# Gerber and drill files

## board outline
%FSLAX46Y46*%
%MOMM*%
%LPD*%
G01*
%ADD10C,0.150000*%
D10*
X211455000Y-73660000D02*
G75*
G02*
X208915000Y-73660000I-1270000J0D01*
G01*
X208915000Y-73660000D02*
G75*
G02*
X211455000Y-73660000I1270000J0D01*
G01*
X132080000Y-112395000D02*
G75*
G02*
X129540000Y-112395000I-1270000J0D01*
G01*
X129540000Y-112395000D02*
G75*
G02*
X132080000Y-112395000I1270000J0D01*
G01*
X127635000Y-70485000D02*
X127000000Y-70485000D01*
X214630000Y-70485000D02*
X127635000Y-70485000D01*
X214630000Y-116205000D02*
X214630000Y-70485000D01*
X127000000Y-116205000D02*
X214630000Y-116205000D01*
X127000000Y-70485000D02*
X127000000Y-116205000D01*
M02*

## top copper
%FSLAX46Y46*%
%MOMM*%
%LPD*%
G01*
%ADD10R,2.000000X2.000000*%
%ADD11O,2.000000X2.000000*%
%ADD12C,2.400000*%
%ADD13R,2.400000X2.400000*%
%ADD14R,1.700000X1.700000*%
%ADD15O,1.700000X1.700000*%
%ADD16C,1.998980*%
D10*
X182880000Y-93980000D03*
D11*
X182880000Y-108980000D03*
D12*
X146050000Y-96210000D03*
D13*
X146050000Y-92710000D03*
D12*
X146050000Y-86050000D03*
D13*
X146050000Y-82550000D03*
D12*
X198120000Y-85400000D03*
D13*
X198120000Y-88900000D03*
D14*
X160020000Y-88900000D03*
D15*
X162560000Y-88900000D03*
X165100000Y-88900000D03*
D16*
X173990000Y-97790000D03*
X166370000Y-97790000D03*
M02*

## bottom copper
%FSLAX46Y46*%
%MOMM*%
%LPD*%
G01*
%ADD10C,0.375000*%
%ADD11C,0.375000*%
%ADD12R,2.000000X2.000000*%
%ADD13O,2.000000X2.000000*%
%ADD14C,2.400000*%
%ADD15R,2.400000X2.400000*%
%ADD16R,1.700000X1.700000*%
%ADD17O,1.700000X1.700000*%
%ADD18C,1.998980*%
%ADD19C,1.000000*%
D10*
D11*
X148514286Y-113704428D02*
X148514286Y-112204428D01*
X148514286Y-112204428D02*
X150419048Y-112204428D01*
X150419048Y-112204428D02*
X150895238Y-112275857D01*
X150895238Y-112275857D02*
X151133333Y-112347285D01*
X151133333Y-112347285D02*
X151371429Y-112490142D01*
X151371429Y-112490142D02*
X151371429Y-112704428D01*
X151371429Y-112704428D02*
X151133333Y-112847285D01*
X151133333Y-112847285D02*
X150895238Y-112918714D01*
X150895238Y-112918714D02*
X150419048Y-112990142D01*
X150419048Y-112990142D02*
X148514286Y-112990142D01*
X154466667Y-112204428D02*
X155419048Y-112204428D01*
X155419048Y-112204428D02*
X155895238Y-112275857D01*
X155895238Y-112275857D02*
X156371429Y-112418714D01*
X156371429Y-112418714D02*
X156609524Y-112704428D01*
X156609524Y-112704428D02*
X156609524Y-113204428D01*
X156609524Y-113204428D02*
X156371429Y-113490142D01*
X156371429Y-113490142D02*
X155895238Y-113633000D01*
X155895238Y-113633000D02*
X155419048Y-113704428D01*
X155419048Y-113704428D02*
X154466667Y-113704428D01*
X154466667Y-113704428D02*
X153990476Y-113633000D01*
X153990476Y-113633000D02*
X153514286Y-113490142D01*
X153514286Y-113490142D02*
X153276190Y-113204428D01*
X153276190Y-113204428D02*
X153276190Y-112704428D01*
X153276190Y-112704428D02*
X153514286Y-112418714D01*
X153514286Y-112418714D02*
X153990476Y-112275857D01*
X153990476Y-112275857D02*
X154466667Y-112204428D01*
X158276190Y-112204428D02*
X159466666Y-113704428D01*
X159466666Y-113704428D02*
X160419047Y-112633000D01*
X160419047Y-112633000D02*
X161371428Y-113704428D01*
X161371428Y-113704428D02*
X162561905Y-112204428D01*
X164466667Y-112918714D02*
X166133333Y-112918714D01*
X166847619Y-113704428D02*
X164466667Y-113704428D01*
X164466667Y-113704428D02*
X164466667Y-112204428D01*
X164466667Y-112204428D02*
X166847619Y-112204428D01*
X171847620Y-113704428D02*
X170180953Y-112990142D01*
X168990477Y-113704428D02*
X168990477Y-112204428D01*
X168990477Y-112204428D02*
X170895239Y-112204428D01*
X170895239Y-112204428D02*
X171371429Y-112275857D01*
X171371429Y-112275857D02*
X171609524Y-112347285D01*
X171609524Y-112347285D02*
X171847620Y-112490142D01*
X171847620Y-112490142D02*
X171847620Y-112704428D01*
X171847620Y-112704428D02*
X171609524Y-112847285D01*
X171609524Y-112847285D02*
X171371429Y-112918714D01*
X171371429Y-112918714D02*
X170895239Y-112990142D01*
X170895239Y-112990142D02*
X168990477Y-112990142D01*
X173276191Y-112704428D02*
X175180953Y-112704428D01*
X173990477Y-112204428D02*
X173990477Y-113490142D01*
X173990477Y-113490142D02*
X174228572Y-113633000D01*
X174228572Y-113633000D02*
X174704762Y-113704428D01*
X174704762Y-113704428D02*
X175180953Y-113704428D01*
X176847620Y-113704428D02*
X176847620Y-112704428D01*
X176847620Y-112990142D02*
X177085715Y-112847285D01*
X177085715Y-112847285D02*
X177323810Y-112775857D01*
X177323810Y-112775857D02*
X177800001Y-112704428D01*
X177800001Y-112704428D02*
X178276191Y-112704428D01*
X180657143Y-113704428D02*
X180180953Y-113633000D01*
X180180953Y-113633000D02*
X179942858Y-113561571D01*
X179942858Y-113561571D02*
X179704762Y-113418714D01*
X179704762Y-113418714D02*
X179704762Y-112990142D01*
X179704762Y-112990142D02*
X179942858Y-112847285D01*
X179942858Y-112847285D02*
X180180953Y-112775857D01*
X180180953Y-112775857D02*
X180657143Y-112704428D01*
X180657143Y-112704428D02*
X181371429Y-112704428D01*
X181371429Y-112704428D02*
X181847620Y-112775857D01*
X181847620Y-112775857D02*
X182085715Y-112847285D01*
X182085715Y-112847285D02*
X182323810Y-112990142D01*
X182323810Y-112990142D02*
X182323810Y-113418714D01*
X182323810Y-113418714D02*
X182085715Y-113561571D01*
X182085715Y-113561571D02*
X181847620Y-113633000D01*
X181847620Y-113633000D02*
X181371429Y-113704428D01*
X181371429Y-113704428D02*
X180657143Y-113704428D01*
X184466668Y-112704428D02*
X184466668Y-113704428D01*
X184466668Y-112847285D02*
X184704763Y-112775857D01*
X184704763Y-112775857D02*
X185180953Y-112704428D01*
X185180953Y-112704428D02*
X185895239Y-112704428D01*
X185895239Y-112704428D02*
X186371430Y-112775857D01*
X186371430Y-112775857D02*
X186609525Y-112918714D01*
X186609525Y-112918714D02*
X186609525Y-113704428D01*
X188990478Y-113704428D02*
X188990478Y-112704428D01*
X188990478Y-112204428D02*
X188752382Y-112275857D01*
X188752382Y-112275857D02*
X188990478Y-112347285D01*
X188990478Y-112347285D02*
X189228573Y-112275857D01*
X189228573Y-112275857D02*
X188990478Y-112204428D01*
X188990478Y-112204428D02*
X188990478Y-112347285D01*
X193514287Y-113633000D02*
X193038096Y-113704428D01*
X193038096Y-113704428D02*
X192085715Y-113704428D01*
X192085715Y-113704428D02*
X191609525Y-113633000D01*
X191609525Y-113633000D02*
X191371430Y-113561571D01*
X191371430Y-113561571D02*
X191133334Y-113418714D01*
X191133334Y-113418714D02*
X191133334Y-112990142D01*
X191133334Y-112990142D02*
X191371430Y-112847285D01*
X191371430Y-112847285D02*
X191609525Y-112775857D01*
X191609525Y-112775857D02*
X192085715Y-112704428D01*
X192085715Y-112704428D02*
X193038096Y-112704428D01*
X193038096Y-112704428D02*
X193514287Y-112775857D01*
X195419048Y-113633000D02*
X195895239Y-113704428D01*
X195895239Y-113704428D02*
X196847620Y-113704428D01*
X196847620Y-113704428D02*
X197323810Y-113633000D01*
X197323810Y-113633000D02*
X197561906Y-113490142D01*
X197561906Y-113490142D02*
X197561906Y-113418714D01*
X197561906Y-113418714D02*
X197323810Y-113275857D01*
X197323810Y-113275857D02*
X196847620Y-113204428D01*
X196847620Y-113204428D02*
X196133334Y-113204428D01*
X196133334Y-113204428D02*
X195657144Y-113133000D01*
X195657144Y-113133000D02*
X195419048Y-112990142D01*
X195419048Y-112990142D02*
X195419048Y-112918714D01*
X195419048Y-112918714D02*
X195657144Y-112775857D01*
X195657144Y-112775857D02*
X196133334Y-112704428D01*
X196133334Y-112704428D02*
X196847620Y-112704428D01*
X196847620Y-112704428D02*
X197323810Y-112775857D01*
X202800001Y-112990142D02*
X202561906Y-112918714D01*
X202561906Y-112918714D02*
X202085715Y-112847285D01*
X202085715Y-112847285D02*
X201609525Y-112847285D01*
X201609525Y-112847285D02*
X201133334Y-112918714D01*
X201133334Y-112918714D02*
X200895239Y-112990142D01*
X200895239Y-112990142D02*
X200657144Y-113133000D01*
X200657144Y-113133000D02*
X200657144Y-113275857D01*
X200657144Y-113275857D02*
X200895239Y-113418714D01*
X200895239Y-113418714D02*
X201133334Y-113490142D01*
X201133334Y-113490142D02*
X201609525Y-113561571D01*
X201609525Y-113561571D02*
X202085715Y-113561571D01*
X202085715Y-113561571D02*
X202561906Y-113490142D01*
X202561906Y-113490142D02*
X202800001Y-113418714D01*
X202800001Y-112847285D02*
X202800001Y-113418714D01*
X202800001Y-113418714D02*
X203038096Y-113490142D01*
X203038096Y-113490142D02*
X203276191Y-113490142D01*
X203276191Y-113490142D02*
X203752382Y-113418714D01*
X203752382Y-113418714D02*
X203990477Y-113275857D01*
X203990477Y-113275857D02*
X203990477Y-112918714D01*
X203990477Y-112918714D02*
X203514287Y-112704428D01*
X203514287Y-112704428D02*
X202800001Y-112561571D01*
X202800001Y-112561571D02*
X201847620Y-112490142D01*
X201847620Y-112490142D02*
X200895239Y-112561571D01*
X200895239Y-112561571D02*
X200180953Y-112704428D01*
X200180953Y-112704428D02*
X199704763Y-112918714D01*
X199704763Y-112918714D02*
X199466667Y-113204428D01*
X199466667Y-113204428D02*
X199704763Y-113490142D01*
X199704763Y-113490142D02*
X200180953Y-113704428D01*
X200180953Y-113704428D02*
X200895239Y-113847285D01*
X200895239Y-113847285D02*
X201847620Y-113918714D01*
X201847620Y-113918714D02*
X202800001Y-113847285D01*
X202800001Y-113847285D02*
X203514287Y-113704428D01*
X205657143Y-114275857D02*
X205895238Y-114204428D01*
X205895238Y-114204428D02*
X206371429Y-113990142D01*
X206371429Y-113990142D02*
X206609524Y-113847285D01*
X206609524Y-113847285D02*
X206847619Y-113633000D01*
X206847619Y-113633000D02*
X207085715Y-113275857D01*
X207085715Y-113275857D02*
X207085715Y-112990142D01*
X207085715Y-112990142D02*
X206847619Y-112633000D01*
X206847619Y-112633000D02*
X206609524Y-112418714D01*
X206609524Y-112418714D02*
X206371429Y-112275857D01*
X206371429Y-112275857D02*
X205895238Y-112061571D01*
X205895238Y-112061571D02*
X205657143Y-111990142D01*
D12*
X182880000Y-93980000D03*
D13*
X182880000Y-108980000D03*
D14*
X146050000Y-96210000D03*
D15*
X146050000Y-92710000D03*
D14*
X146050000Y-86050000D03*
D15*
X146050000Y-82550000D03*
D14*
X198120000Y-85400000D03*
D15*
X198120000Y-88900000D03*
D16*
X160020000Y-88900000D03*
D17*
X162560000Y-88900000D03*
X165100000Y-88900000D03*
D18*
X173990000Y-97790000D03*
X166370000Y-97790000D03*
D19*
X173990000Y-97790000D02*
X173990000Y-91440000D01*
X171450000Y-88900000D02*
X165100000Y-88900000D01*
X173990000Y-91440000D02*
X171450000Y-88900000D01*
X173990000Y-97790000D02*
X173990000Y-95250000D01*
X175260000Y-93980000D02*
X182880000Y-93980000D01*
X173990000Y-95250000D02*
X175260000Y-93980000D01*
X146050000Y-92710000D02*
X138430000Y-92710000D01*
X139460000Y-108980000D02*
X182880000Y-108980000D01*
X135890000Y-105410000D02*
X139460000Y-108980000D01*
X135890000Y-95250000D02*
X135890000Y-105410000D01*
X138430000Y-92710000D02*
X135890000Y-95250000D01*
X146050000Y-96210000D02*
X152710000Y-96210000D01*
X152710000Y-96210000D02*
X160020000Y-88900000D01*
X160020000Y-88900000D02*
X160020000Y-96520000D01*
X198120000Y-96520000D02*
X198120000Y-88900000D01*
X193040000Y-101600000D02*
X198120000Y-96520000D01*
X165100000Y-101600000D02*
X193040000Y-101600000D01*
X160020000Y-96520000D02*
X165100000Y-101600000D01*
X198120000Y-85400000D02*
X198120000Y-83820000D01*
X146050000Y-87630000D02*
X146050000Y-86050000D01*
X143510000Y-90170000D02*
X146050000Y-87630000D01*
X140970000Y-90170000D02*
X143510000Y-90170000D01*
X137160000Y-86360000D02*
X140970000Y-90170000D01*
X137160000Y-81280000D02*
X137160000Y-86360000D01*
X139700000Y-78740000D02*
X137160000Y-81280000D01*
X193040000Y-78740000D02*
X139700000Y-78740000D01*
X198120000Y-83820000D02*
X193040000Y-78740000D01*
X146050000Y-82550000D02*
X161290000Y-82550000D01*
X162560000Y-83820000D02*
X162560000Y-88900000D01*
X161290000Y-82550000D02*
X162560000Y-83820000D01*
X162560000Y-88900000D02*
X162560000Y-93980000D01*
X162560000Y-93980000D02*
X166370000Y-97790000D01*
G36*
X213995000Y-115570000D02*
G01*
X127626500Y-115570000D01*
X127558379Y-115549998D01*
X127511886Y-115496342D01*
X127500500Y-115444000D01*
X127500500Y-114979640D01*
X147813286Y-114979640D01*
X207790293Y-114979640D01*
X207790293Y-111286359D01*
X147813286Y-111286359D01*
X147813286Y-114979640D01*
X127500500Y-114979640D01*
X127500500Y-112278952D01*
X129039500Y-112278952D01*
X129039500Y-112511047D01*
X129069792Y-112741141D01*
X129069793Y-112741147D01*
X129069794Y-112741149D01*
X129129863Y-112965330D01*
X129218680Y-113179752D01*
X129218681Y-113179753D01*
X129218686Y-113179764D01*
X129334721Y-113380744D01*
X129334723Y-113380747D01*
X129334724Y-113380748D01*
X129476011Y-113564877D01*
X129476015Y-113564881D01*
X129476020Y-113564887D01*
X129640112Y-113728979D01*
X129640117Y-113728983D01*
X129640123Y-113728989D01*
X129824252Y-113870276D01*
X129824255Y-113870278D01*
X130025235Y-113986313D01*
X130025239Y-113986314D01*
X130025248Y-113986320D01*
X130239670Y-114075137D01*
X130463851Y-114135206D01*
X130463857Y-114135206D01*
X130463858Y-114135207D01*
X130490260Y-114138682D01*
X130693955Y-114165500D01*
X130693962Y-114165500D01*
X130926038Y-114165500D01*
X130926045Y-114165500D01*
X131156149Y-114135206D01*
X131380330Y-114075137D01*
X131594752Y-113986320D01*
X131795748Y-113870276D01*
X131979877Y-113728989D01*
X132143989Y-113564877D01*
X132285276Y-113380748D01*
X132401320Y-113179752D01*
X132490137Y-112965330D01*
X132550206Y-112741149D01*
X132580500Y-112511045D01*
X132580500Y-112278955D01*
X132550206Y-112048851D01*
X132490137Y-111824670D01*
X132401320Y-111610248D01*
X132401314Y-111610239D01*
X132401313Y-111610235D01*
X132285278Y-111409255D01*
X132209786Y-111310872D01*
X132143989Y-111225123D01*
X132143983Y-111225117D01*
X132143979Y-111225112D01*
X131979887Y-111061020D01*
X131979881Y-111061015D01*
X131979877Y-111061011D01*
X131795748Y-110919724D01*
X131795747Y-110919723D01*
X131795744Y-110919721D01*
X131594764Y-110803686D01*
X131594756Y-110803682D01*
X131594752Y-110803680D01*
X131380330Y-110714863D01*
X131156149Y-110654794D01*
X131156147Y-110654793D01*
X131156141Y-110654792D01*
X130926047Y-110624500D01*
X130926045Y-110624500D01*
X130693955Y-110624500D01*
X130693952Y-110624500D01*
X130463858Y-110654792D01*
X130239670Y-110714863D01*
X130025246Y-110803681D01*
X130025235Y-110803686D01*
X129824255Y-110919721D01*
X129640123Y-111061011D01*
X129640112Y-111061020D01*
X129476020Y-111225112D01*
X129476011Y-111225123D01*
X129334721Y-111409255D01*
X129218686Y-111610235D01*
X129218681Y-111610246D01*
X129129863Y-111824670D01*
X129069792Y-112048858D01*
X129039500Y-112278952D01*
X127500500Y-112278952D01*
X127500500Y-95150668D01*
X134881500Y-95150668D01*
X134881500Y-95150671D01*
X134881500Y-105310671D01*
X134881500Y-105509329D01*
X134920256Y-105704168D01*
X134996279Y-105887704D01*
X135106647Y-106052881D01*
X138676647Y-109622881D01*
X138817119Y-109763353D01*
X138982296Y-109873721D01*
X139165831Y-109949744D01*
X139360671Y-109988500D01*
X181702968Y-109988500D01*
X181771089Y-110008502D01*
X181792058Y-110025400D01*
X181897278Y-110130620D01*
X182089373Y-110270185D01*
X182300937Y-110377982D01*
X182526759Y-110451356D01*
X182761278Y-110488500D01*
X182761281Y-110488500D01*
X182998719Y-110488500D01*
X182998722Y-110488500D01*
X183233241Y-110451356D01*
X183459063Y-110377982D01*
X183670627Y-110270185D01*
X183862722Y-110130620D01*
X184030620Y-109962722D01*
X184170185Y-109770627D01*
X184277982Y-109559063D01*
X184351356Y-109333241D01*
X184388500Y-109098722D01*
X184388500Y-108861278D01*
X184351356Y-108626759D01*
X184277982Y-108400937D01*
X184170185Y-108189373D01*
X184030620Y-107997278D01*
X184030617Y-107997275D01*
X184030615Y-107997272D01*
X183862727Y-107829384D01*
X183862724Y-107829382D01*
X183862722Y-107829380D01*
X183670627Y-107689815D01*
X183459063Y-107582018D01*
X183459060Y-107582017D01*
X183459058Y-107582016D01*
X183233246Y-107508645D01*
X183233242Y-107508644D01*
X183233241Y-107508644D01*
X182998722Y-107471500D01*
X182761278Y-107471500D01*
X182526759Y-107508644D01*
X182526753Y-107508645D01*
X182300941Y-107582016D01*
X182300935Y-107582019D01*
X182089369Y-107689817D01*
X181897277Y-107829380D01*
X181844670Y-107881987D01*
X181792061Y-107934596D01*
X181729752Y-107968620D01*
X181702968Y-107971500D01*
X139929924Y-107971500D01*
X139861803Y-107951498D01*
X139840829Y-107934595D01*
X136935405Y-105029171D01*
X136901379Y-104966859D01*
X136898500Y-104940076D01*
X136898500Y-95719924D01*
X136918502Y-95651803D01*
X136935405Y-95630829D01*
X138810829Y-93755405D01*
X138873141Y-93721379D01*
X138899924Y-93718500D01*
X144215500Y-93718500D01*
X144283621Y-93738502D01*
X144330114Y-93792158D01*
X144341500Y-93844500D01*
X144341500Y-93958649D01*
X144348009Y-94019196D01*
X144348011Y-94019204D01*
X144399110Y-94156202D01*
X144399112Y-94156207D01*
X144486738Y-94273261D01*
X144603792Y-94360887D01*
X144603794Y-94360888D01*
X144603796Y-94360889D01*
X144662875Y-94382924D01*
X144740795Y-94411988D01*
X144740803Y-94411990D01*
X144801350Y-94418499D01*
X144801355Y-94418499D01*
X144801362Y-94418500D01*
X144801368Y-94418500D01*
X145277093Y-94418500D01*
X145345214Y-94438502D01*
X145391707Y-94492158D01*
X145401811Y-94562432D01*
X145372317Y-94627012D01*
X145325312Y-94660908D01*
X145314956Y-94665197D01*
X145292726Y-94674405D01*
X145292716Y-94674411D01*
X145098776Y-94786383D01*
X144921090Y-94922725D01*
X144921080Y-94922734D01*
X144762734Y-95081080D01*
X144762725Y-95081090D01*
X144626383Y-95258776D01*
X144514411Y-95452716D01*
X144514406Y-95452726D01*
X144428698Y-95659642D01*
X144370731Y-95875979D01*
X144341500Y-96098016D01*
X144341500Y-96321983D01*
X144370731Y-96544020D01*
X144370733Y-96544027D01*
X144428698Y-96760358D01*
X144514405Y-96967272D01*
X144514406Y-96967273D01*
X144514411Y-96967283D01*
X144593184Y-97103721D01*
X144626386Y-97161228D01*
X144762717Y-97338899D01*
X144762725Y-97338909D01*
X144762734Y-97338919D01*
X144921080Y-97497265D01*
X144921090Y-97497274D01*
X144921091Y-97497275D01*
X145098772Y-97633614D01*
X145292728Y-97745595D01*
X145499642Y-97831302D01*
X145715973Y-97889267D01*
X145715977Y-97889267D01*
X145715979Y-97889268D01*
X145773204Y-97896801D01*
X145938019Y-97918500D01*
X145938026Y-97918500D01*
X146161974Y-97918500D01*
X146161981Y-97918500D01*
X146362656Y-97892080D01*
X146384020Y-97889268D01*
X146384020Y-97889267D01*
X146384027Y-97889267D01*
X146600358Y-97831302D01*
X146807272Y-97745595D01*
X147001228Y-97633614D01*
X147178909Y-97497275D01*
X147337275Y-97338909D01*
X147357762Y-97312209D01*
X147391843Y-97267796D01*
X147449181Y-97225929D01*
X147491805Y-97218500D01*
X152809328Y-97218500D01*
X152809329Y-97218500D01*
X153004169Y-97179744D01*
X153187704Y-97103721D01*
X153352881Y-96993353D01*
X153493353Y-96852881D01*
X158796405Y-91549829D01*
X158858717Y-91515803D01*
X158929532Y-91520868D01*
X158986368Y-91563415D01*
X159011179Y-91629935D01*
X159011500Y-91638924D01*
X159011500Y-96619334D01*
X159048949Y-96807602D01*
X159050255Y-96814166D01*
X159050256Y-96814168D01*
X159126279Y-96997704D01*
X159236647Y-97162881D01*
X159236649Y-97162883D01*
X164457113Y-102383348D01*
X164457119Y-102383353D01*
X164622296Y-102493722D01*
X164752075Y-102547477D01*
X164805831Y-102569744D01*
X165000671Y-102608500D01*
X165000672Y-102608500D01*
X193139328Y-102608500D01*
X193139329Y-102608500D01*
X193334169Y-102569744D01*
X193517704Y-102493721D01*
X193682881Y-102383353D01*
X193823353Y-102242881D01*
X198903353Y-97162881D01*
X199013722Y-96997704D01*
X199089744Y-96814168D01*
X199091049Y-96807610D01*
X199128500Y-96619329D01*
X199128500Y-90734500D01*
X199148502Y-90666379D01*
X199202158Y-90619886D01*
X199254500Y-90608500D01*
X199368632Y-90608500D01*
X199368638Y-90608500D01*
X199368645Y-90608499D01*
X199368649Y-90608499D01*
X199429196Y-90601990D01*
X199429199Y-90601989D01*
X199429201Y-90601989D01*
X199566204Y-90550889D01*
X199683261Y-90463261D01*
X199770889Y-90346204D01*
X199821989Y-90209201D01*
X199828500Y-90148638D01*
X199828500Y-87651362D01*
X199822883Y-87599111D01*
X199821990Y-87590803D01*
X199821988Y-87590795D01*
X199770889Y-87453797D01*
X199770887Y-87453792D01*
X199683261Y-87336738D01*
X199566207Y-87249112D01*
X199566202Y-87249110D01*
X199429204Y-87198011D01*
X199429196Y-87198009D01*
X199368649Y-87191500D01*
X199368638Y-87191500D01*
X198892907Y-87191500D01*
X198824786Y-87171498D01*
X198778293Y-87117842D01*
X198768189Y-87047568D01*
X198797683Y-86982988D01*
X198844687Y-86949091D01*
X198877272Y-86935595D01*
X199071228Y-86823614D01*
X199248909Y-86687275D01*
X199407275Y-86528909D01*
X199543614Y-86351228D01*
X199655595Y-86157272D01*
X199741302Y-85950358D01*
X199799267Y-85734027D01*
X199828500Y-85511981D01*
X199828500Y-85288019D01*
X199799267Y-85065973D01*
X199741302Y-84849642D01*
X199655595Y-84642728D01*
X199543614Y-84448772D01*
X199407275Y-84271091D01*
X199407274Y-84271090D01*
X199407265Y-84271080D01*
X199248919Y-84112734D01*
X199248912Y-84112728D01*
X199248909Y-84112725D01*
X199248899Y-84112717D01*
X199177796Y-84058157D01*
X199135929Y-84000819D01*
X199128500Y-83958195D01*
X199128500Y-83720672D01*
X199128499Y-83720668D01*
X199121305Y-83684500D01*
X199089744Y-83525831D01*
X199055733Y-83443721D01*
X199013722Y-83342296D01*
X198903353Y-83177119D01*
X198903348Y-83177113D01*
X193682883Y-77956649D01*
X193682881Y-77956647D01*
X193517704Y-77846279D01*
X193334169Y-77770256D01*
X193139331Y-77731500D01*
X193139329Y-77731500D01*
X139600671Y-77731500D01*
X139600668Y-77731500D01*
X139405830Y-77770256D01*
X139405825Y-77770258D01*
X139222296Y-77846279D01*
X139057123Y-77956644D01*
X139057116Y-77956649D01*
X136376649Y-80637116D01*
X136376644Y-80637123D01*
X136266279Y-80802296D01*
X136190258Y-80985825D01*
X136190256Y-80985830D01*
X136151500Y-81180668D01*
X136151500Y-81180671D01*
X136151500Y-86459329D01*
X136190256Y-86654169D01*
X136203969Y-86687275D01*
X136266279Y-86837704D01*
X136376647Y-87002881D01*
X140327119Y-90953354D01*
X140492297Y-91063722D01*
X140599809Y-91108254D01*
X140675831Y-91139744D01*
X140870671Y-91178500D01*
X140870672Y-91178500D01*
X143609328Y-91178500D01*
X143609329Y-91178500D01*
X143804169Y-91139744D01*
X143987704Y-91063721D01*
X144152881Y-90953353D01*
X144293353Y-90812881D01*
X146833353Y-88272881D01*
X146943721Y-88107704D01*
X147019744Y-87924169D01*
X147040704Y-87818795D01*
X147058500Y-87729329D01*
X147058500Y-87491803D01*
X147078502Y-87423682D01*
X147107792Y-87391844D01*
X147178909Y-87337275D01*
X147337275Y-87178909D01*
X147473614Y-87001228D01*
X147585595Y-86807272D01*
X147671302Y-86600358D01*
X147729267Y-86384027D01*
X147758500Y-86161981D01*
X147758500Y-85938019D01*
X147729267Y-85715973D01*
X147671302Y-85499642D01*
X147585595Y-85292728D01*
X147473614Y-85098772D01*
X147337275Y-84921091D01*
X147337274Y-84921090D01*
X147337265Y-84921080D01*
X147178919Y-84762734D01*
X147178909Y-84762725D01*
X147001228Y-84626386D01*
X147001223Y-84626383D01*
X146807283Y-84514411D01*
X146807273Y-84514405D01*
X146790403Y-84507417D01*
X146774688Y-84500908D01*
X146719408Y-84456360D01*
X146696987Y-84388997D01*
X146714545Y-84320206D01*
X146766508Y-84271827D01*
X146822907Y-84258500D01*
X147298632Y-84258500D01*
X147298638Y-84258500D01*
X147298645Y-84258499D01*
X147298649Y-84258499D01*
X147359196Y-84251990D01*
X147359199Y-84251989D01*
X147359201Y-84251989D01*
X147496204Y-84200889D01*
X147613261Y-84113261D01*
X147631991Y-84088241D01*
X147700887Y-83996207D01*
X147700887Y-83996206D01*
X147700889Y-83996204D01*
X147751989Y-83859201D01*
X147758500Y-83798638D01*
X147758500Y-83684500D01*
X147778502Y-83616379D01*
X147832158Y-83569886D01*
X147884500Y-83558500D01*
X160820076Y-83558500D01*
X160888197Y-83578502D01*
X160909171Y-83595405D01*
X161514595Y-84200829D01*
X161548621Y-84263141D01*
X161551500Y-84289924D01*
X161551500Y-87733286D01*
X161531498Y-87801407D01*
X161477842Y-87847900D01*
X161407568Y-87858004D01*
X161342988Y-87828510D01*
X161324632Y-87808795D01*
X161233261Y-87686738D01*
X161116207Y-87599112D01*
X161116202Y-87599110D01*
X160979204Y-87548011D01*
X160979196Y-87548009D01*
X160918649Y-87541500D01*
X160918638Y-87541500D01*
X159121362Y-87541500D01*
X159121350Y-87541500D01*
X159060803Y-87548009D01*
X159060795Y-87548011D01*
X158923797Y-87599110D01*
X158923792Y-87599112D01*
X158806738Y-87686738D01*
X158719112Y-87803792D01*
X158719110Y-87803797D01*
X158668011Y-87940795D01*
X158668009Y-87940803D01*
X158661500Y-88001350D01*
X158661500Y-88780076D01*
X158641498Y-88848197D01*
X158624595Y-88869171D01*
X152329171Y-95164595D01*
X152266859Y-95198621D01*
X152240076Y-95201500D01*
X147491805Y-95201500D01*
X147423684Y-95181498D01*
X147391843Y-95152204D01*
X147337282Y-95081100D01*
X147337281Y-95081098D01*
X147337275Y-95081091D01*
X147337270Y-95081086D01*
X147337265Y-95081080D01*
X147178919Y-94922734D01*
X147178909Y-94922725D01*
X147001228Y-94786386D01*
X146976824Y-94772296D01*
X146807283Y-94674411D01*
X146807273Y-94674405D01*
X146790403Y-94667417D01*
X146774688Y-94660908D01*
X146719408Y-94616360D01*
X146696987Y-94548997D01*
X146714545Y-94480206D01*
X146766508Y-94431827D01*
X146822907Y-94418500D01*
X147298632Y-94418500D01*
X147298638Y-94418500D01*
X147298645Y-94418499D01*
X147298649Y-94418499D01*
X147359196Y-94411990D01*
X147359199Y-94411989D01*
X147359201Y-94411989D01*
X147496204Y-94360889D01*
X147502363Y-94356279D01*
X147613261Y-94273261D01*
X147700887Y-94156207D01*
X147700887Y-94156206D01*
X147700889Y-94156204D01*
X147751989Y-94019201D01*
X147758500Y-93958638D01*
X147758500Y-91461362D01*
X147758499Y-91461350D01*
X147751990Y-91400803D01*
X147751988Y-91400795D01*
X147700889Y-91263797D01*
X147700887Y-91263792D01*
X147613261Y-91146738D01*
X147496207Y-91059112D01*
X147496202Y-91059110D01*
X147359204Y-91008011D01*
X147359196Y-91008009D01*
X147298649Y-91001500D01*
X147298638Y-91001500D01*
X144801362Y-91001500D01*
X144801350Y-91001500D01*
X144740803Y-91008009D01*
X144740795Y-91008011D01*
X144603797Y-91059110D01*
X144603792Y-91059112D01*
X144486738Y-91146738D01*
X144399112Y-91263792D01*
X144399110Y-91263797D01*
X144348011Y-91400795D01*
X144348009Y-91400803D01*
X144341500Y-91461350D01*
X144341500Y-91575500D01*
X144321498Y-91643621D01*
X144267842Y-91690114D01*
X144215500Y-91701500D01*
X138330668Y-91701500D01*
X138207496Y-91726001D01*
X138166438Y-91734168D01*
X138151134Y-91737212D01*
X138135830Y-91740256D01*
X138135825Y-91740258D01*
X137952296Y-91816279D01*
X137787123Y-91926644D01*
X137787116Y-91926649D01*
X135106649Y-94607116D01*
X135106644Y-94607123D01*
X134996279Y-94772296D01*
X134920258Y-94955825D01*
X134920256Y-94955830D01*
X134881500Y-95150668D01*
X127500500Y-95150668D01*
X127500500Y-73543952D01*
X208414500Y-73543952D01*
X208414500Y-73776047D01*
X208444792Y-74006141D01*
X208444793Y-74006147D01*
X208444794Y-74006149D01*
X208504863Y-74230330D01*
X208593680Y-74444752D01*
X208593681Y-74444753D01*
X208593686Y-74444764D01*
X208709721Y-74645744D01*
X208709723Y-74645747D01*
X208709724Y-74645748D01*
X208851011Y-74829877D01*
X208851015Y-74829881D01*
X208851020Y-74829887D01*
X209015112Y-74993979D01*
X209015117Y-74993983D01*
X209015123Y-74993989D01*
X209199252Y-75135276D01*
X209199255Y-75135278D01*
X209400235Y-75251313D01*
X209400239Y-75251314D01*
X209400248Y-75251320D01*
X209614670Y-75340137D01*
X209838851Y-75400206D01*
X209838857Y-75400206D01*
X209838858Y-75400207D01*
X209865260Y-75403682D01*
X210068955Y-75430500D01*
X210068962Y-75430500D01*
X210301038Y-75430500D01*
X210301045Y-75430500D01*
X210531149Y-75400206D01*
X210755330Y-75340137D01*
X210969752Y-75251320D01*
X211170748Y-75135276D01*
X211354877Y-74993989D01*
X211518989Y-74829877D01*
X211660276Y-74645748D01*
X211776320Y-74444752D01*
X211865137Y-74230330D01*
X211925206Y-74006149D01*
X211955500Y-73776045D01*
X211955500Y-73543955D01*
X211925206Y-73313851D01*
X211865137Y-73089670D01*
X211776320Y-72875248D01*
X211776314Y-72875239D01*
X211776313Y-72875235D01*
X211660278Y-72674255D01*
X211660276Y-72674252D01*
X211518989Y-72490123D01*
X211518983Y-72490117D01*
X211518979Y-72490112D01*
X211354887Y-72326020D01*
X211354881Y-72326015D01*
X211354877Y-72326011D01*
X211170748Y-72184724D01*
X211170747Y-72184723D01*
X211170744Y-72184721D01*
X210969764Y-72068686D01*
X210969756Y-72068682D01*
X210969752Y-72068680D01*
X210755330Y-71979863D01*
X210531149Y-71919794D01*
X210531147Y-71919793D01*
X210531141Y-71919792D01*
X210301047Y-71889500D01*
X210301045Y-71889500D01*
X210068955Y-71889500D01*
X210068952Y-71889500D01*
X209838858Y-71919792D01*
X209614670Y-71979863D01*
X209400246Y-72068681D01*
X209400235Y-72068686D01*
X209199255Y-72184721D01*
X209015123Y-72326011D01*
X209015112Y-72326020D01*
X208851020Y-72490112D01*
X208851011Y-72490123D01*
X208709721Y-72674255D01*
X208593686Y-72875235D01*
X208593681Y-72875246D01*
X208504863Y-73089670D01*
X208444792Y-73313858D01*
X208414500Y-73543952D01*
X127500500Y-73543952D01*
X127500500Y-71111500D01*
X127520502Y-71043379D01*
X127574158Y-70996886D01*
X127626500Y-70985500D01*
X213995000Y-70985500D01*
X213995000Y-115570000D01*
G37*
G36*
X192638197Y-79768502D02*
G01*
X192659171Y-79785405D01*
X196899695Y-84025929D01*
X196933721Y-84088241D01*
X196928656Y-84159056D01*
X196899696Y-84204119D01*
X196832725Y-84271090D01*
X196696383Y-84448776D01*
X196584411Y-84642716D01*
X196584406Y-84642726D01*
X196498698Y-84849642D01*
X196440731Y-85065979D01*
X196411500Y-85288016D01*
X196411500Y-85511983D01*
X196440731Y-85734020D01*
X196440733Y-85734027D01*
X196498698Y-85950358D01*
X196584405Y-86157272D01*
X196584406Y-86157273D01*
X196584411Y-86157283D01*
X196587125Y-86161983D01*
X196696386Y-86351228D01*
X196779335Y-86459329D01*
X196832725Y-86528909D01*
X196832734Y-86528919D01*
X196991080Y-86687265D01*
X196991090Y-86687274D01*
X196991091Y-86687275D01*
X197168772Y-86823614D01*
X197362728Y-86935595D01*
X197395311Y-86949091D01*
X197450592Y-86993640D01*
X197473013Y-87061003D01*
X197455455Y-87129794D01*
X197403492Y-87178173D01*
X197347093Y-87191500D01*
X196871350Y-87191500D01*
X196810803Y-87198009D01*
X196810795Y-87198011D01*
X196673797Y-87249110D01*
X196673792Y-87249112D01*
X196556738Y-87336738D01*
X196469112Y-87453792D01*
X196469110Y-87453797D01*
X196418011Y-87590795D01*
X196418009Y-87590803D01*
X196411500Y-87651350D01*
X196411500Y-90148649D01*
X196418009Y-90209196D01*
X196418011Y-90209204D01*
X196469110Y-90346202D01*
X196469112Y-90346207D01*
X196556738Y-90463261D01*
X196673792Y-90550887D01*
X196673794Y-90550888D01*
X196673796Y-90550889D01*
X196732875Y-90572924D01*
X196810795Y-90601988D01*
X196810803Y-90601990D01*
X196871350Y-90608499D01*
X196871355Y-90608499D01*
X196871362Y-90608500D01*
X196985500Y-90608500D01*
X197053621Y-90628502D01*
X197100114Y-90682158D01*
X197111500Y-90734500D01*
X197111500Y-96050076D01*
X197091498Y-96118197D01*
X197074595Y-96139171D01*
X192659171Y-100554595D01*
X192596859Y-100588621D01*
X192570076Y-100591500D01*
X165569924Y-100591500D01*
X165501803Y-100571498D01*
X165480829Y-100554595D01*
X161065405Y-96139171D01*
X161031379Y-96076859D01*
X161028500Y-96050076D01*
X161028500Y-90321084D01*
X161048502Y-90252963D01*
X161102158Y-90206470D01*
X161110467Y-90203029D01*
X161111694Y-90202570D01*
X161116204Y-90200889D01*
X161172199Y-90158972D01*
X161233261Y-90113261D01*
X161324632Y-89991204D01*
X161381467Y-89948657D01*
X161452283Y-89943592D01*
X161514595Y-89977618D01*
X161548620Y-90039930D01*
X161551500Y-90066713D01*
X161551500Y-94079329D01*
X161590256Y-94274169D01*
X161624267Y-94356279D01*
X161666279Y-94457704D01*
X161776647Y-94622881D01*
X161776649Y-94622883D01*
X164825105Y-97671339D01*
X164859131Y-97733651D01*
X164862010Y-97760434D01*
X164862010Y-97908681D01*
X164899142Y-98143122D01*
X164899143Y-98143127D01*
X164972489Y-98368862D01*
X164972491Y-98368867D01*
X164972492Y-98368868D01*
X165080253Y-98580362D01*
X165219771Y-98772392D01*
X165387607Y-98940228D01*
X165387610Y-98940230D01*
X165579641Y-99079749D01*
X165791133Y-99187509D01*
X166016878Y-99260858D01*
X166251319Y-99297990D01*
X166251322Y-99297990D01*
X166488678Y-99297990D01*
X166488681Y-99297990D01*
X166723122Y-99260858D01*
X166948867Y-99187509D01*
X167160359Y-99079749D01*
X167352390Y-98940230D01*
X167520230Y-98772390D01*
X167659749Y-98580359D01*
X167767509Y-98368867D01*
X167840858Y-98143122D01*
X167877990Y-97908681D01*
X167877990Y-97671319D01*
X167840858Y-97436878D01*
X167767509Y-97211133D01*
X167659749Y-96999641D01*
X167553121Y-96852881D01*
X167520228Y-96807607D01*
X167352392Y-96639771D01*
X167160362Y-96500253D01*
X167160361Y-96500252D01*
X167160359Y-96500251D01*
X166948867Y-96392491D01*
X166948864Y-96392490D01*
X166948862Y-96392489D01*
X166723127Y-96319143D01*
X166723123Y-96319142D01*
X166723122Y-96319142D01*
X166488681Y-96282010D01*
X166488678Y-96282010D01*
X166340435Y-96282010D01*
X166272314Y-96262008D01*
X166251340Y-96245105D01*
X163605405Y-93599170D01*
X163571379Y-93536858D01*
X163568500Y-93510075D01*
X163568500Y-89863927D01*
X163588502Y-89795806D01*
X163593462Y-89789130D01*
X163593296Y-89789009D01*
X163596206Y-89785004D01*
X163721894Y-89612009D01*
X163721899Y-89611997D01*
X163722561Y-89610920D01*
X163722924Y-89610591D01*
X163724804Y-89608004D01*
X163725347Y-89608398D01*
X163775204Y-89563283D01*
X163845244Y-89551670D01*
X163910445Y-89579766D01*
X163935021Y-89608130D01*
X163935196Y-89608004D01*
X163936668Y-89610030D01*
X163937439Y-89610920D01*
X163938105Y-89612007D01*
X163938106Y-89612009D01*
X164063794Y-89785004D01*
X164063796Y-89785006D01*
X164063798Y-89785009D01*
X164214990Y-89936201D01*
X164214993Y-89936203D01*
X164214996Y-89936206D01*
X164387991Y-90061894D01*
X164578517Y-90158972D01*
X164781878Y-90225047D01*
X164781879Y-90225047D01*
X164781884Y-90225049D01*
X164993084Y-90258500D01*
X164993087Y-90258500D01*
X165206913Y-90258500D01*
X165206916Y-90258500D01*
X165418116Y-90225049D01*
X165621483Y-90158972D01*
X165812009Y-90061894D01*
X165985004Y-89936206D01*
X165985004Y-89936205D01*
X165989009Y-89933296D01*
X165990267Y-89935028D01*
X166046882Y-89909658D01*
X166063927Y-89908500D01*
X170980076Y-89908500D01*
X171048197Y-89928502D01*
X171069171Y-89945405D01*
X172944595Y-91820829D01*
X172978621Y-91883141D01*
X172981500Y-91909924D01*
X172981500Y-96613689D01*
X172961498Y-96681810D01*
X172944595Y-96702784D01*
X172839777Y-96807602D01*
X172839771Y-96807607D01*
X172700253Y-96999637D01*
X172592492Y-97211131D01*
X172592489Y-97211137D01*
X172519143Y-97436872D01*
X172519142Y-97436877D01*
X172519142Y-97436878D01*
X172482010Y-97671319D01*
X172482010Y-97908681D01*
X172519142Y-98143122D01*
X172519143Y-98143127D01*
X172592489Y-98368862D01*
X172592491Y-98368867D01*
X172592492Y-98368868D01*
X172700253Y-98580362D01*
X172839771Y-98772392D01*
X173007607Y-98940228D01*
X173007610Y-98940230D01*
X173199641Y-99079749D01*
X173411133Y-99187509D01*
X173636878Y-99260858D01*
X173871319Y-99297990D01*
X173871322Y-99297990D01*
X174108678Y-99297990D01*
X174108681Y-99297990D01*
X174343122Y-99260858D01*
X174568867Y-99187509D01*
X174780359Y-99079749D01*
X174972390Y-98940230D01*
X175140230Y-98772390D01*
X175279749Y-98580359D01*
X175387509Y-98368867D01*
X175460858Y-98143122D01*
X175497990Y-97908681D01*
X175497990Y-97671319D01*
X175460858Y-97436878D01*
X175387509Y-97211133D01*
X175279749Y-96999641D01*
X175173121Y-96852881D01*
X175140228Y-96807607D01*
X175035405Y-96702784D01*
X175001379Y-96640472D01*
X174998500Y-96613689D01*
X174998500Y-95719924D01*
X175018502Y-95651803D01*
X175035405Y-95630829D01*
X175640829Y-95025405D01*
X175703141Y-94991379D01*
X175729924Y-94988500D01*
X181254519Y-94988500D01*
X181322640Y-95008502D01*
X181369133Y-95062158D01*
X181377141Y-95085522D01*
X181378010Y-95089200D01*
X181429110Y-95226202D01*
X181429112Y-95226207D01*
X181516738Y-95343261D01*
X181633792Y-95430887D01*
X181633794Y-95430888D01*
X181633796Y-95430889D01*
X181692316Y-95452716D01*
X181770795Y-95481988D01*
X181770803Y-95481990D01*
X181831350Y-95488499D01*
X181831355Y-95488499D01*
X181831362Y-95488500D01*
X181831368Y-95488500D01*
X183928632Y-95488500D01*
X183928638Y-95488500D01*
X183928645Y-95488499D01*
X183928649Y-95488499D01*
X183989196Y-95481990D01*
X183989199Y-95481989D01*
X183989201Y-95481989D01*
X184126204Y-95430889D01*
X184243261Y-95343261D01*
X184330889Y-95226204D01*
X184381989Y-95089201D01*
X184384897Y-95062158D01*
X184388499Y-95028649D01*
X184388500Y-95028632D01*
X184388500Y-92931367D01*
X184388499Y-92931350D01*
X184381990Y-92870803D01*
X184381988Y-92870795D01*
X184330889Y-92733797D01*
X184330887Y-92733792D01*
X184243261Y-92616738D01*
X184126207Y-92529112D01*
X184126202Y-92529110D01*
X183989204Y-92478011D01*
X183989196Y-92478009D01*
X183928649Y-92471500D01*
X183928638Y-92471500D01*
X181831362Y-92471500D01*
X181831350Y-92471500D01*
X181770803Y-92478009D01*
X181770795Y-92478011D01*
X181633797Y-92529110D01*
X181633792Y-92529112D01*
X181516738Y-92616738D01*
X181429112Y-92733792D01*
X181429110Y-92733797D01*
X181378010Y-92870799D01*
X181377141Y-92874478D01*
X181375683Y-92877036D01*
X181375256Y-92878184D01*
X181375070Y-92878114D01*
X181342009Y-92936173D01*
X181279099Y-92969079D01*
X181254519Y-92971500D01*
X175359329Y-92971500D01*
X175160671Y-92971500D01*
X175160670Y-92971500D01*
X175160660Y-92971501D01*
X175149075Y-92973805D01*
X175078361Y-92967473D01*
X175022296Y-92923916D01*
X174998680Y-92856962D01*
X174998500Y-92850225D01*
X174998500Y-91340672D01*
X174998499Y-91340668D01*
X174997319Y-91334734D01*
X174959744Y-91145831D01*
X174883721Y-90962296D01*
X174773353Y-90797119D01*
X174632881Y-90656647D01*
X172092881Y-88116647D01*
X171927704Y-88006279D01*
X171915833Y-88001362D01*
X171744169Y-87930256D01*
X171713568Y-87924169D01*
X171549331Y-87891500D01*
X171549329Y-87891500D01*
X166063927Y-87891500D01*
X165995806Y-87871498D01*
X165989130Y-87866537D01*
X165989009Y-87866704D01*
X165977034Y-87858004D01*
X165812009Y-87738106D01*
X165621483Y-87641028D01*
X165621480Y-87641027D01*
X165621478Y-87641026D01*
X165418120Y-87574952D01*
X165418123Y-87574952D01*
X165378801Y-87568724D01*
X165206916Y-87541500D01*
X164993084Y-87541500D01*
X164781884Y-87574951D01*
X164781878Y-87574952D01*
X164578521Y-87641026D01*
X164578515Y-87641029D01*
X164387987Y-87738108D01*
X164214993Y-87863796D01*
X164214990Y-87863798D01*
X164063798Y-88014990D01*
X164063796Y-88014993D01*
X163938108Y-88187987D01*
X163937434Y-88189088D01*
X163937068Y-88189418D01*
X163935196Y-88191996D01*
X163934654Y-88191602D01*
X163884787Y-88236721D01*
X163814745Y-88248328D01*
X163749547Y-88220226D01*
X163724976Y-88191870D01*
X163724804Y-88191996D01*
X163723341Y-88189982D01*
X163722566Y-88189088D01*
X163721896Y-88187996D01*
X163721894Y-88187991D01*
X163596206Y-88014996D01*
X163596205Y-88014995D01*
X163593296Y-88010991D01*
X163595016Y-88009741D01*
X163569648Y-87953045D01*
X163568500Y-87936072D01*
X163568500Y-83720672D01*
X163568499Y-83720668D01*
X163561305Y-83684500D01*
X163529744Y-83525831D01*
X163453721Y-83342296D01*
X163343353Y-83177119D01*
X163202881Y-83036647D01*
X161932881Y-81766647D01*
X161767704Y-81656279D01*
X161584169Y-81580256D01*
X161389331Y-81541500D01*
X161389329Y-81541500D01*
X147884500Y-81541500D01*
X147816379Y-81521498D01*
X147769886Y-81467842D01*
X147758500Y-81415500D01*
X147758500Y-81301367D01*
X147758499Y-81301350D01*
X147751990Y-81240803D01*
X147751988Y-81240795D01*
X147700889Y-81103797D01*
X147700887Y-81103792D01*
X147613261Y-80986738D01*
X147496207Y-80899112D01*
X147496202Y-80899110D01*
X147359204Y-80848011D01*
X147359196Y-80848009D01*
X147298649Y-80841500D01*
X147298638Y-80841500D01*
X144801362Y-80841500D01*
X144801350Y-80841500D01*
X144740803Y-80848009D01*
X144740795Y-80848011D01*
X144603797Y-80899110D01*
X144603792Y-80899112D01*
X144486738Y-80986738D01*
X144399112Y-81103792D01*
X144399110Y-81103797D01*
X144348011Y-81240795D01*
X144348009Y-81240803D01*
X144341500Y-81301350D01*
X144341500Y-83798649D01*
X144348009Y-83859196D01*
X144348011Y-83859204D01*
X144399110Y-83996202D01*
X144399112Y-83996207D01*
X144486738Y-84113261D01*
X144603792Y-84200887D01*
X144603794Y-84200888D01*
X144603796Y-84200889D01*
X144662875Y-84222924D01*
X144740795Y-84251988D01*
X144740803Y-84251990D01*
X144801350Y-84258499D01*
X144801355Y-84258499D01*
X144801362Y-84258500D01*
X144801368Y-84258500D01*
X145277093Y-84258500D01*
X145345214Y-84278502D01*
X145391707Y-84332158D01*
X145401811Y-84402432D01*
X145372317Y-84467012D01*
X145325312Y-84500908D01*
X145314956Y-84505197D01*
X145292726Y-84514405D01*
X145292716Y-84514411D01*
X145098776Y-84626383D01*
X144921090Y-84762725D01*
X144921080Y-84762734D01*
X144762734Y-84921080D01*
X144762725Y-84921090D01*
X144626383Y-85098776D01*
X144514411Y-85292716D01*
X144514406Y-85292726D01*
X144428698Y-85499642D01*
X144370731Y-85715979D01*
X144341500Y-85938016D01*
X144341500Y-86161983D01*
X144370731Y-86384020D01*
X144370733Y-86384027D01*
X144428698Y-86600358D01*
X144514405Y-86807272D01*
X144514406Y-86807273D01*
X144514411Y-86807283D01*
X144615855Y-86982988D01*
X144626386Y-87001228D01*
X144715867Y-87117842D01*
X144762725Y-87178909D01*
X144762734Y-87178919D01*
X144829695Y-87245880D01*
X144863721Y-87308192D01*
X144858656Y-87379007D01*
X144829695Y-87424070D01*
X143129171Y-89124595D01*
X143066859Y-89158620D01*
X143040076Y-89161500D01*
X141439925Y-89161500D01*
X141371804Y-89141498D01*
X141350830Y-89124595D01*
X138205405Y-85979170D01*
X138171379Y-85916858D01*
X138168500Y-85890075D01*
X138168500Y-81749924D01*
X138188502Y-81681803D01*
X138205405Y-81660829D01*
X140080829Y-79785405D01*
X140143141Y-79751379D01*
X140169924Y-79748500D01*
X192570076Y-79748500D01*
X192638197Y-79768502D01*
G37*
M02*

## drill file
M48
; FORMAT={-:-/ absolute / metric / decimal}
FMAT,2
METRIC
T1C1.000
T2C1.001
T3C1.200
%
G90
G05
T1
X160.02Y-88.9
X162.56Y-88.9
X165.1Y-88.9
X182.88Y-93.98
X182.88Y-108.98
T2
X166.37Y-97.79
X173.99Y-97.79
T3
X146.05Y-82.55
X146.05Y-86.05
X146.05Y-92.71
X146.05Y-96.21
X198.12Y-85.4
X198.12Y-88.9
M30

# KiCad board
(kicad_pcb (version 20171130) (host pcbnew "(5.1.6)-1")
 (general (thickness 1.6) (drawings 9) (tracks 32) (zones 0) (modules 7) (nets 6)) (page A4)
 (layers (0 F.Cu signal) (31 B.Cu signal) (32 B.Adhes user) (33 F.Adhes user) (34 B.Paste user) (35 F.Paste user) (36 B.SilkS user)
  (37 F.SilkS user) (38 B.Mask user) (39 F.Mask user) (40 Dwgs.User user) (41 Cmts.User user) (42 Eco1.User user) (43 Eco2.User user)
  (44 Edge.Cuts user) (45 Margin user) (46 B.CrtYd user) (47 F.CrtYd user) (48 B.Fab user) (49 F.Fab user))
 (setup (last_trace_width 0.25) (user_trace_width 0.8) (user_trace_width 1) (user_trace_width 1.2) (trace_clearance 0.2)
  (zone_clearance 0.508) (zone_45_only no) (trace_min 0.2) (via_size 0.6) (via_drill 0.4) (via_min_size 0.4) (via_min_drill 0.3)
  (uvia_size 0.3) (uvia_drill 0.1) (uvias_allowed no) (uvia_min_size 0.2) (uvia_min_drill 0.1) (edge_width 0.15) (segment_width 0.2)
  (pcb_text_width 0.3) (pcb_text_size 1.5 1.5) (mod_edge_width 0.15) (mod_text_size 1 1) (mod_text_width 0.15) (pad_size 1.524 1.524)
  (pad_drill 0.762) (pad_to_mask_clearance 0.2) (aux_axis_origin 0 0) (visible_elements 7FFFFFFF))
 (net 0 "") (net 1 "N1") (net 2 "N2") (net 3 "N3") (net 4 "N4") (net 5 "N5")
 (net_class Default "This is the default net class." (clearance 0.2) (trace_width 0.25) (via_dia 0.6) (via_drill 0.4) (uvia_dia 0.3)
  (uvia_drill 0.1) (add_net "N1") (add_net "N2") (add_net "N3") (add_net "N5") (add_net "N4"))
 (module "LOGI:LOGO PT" (layer F.Cu) (at 181.61 81.28)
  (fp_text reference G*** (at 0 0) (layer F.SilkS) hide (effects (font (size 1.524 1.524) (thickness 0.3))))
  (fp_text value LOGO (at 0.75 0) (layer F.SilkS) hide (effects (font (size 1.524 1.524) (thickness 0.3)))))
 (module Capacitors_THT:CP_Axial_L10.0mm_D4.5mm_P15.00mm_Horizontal (layer F.Cu) (at 182.88 93.98 270)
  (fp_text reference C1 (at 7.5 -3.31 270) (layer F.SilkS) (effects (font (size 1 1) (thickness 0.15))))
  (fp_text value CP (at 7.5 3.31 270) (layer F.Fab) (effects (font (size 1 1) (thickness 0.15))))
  (pad 1 thru_hole rect (at 0 0 270) (size 2 2) (drill 1) (layers *.Cu *.Mask) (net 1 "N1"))
  (pad 2 thru_hole oval (at 15 0 270) (size 2 2) (drill 1) (layers *.Cu *.Mask) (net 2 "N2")))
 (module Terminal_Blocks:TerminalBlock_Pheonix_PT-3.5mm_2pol (layer F.Cu) (at 146.05 92.71 270)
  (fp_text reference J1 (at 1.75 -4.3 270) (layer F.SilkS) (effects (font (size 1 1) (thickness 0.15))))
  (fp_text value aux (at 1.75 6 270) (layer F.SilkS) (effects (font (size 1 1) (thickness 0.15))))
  (pad 2 thru_hole circle (at 3.5 0 270) (size 2.4 2.4) (drill 1.2) (layers *.Cu *.Mask) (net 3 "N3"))
  (pad 1 thru_hole rect (at 0 0 270) (size 2.4 2.4) (drill 1.2) (layers *.Cu *.Mask) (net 2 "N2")))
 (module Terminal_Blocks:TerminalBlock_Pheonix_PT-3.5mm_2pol (layer F.Cu) (at 146.05 82.55 270)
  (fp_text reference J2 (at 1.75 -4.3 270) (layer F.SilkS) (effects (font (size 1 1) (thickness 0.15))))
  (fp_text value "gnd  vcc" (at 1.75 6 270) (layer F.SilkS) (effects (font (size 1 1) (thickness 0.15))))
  (pad 2 thru_hole circle (at 3.5 0 270) (size 2.4 2.4) (drill 1.2) (layers *.Cu *.Mask) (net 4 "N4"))
  (pad 1 thru_hole rect (at 0 0 270) (size 2.4 2.4) (drill 1.2) (layers *.Cu *.Mask) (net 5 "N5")))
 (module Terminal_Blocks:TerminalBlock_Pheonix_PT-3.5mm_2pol (layer F.Cu) (at 198.12 88.9 90)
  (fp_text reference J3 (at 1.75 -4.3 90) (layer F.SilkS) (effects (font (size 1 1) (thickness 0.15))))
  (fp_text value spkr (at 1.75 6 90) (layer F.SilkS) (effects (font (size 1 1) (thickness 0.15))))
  (pad 2 thru_hole circle (at 3.5 0 90) (size 2.4 2.4) (drill 1.2) (layers *.Cu *.Mask) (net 4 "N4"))
  (pad 1 thru_hole rect (at 0 0 90) (size 2.4 2.4) (drill 1.2) (layers *.Cu *.Mask) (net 3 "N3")))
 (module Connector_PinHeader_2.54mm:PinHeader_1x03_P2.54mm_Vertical (layer F.Cu) (at 160.02 88.9 90)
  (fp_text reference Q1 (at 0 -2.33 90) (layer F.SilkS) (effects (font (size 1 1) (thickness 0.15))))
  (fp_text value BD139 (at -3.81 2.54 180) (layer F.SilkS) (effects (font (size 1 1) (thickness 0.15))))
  (pad 1 thru_hole rect (at 0 0 90) (size 1.7 1.7) (drill 1) (layers *.Cu *.Mask) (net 3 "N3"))
  (pad 2 thru_hole oval (at 0 2.54 90) (size 1.7 1.7) (drill 1) (layers *.Cu *.Mask) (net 5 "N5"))
  (pad 3 thru_hole oval (at 0 5.08 90) (size 1.7 1.7) (drill 1) (layers *.Cu *.Mask) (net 1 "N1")))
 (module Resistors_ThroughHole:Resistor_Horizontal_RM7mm (layer F.Cu) (at 173.99 97.79 180)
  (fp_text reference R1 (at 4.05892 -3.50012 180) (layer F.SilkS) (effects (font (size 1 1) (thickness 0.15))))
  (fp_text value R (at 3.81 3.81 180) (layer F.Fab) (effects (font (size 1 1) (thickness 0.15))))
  (pad 1 thru_hole circle (at 0 0 180) (size 1.99898 1.99898) (drill 1.00076) (layers *.Cu *.SilkS *.Mask) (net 1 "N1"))
  (pad 2 thru_hole circle (at 7.62 0 180) (size 1.99898 1.99898) (drill 1.00076) (layers *.Cu *.SilkS *.Mask) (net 5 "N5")))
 (gr_circle (center 210.185 73.66) (end 210.185 72.39) (layer Edge.Cuts) (width 0.15))
 (gr_circle (center 130.81 112.395) (end 130.81 111.125) (layer Edge.Cuts) (width 0.15))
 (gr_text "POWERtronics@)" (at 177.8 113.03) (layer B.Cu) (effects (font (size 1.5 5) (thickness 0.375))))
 (gr_line (start 127.635 70.485) (end 127 70.485) (angle 90) (layer Edge.Cuts) (width 0.15))
 (gr_line (start 214.63 70.485) (end 127.635 70.485) (angle 90) (layer Edge.Cuts) (width 0.15))
 (gr_line (start 214.63 116.205) (end 214.63 70.485) (angle 90) (layer Edge.Cuts) (width 0.15))
 (gr_line (start 127 116.205) (end 214.63 116.205) (angle 90) (layer Edge.Cuts) (width 0.15))
 (gr_line (start 127 70.485) (end 127 116.205) (angle 90) (layer Edge.Cuts) (width 0.15))
 (segment (start 173.99 97.79) (end 173.99 91.44) (width 1) (layer B.Cu) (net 1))
 (segment (start 171.45 88.9) (end 165.1 88.9) (width 1) (layer B.Cu) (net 1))
 (segment (start 173.99 91.44) (end 171.45 88.9) (width 1) (layer B.Cu) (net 1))
 (segment (start 173.99 97.79) (end 173.99 95.25) (width 1) (layer B.Cu) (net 1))
 (segment (start 175.26 93.98) (end 182.88 93.98) (width 1) (layer B.Cu) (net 1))
 (segment (start 173.99 95.25) (end 175.26 93.98) (width 1) (layer B.Cu) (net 1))
 (segment (start 146.05 92.71) (end 138.43 92.71) (width 1) (layer B.Cu) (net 2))
 (segment (start 139.46 108.98) (end 182.88 108.98) (width 1) (layer B.Cu) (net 2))
 (segment (start 135.89 105.41) (end 139.46 108.98) (width 1) (layer B.Cu) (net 2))
 (segment (start 135.89 95.25) (end 135.89 105.41) (width 1) (layer B.Cu) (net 2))
 (segment (start 138.43 92.71) (end 135.89 95.25) (width 1) (layer B.Cu) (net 2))
 (segment (start 146.05 96.21) (end 152.71 96.21) (width 1) (layer B.Cu) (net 3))
 (segment (start 152.71 96.21) (end 160.02 88.9) (width 1) (layer B.Cu) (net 3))
 (segment (start 160.02 88.9) (end 160.02 96.52) (width 1) (layer B.Cu) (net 3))
 (segment (start 198.12 96.52) (end 198.12 88.9) (width 1) (layer B.Cu) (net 3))
 (segment (start 193.04 101.6) (end 198.12 96.52) (width 1) (layer B.Cu) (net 3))
 (segment (start 165.1 101.6) (end 193.04 101.6) (width 1) (layer B.Cu) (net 3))
 (segment (start 160.02 96.52) (end 165.1 101.6) (width 1) (layer B.Cu) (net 3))
 (segment (start 198.12 85.4) (end 198.12 83.82) (width 1) (layer B.Cu) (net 4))
 (segment (start 146.05 87.63) (end 146.05 86.05) (width 1) (layer B.Cu) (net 4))
 (segment (start 143.51 90.17) (end 146.05 87.63) (width 1) (layer B.Cu) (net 4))
 (segment (start 140.97 90.17) (end 143.51 90.17) (width 1) (layer B.Cu) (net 4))
 (segment (start 137.16 86.36) (end 140.97 90.17) (width 1) (layer B.Cu) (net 4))
 (segment (start 137.16 81.28) (end 137.16 86.36) (width 1) (layer B.Cu) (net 4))
 (segment (start 139.7 78.74) (end 137.16 81.28) (width 1) (layer B.Cu) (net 4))
 (segment (start 193.04 78.74) (end 139.7 78.74) (width 1) (layer B.Cu) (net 4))
 (segment (start 198.12 83.82) (end 193.04 78.74) (width 1) (layer B.Cu) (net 4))
 (segment (start 146.05 82.55) (end 161.29 82.55) (width 1) (layer B.Cu) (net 5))
 (segment (start 162.56 83.82) (end 162.56 88.9) (width 1) (layer B.Cu) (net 5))
 (segment (start 161.29 82.55) (end 162.56 83.82) (width 1) (layer B.Cu) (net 5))
 (segment (start 162.56 88.9) (end 162.56 93.98) (width 1) (layer B.Cu) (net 5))
 (segment (start 162.56 93.98) (end 166.37 97.79) (width 1) (layer B.Cu) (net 5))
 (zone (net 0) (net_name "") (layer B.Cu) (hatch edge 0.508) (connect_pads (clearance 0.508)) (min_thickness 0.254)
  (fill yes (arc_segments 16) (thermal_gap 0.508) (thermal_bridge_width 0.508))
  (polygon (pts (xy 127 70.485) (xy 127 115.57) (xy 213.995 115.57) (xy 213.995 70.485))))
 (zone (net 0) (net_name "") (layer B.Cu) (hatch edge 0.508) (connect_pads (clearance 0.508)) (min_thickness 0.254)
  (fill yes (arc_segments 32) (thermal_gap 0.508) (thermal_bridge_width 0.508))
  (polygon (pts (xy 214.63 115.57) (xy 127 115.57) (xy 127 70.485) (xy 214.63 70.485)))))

